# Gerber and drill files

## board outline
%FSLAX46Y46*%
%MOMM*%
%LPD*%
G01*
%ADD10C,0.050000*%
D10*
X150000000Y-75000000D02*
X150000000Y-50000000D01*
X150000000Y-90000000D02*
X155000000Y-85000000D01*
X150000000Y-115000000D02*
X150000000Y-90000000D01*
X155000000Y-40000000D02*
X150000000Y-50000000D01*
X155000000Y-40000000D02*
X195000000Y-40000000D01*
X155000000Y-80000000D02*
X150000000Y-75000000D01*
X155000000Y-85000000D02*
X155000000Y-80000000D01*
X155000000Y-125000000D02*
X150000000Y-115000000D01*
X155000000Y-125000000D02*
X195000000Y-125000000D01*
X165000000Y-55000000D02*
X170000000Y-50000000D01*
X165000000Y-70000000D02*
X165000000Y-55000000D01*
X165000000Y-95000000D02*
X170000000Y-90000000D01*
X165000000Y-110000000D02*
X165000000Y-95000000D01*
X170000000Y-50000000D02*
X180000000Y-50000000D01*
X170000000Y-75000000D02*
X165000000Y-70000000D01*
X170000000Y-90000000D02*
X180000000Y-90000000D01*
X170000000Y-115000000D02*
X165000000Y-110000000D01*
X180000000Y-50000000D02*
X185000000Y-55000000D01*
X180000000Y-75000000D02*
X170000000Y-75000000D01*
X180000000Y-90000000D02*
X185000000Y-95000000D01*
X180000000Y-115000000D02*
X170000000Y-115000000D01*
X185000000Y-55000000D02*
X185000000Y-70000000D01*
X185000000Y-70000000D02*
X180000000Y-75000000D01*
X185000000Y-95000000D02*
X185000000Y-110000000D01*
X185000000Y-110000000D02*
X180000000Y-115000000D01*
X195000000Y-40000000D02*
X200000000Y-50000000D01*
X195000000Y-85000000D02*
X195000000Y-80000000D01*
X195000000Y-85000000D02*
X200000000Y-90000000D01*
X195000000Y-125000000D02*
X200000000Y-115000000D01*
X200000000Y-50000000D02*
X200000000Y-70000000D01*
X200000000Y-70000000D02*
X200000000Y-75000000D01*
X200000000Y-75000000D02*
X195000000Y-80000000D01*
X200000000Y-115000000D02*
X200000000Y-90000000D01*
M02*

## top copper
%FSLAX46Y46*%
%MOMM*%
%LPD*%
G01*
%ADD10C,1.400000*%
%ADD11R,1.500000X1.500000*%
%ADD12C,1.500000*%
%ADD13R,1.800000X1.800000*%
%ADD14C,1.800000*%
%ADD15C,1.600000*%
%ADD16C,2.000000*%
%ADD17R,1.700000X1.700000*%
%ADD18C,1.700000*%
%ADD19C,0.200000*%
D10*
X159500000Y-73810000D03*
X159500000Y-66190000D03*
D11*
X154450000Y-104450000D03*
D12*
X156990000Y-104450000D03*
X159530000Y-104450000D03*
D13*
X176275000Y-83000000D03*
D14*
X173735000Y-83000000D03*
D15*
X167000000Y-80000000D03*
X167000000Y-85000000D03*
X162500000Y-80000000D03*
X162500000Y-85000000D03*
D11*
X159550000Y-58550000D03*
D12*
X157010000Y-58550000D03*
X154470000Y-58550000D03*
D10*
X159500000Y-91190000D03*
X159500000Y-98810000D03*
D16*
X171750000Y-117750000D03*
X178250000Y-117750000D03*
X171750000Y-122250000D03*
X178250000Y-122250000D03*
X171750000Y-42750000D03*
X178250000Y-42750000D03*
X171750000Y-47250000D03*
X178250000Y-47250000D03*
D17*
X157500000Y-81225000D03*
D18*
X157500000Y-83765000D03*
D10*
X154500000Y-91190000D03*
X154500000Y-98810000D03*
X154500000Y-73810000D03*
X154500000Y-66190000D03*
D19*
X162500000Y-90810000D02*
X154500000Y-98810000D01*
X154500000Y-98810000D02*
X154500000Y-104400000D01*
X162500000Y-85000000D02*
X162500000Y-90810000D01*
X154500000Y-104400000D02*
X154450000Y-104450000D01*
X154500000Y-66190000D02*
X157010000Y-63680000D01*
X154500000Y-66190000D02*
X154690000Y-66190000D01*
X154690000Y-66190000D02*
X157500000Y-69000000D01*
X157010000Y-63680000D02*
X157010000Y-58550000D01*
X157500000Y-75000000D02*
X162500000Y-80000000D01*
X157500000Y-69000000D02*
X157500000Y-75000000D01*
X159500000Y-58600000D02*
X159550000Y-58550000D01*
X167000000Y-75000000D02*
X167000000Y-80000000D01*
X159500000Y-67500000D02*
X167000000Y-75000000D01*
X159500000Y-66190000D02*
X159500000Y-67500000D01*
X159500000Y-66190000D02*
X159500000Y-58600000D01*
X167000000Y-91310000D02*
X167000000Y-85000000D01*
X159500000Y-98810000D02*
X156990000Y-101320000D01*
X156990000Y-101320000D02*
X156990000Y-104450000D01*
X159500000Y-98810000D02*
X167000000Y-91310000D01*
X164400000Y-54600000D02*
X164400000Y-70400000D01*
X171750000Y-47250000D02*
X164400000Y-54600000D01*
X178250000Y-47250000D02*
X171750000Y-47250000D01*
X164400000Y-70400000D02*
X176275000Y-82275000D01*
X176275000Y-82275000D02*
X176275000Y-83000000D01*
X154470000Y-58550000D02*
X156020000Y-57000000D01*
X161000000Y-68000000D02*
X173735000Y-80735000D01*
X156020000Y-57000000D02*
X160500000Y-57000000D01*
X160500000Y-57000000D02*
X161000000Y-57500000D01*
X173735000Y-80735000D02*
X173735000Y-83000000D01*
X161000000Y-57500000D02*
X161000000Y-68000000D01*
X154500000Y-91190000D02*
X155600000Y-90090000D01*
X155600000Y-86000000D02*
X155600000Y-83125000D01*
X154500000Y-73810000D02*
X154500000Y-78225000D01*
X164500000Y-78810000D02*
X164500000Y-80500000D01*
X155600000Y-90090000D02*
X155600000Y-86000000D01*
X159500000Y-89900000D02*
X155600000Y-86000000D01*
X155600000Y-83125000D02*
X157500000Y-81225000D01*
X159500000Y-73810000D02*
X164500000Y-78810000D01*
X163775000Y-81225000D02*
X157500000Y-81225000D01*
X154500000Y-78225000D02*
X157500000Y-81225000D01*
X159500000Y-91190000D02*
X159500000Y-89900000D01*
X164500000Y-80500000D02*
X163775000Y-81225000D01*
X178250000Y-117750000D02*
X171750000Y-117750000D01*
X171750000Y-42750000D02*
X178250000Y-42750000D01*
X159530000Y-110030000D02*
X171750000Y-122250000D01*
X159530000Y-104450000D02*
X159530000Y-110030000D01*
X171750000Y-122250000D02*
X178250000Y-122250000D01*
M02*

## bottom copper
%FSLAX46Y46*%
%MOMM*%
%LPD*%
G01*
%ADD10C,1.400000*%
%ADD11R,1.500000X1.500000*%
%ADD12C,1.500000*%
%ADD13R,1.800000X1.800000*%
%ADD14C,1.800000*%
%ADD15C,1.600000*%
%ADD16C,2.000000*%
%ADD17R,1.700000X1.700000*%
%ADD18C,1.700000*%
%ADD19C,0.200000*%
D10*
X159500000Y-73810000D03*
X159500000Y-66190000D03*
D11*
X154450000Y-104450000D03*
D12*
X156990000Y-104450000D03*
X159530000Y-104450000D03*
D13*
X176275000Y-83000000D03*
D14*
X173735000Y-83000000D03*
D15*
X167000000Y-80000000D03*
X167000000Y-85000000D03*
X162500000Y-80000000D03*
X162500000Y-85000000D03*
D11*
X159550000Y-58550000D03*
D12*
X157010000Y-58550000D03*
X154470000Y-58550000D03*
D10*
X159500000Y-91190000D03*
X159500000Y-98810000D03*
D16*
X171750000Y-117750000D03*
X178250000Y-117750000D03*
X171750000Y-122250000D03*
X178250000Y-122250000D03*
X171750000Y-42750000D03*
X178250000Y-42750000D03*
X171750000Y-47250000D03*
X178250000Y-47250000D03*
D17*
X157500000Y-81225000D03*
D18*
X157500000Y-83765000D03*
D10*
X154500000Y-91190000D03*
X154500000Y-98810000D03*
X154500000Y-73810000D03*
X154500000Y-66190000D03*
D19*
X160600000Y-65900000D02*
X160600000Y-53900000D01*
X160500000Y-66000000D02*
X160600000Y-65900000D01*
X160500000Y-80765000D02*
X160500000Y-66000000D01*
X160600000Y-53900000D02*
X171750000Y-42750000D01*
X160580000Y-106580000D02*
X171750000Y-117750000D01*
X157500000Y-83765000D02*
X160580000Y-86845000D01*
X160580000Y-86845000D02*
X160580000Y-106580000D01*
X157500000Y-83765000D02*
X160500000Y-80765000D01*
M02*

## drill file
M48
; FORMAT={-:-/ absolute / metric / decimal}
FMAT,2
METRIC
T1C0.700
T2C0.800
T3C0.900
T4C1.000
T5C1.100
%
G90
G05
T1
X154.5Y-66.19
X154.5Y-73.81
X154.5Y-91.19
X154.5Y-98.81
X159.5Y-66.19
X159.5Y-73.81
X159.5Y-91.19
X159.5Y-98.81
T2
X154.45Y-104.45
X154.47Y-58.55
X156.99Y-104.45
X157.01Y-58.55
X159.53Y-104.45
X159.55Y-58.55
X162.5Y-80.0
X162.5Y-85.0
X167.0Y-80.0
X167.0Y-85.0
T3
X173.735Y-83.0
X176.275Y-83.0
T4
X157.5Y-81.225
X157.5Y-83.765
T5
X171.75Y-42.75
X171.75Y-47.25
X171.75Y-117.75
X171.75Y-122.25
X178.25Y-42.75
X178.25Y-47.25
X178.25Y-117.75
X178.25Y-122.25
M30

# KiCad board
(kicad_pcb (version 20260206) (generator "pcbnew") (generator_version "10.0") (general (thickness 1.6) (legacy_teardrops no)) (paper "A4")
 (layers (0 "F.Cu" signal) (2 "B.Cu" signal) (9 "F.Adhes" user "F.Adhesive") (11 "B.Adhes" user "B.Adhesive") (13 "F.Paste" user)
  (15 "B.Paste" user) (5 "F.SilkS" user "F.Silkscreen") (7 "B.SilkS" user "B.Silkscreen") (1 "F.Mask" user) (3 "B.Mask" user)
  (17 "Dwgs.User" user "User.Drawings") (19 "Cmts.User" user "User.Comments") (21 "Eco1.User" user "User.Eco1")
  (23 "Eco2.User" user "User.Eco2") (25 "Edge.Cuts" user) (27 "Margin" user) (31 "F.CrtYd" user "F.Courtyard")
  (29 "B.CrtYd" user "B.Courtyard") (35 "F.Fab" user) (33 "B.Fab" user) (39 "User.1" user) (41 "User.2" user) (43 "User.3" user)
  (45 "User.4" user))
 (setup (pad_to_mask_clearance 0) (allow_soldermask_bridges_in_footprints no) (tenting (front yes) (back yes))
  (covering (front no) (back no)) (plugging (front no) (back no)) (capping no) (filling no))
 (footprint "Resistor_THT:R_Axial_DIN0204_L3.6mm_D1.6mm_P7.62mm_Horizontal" (layer "F.Cu") (at 159.5 73.81 90)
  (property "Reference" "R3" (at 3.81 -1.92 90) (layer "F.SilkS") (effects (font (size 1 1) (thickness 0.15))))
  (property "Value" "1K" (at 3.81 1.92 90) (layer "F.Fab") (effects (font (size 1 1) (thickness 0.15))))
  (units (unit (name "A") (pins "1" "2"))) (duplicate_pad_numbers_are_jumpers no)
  (pad "1" thru_hole circle (at 0 0 90) (size 1.4 1.4) (drill 0.7) (layers "*.Cu" "*.Mask") (remove_unused_layers no) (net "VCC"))
  (pad "2" thru_hole circle (at 7.62 0 90) (size 1.4 1.4) (drill 0.7) (layers "*.Cu" "*.Mask") (remove_unused_layers no) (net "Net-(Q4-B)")))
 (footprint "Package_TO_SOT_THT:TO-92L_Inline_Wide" (layer "F.Cu") (at 154.45 104.45)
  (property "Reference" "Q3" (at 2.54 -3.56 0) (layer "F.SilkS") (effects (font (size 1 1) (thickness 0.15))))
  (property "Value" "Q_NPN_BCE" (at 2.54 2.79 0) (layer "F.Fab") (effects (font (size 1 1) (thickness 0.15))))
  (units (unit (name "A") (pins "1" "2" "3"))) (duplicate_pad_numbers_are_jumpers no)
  (pad "1" thru_hole rect (at 0 0) (size 1.5 1.5) (drill 0.8) (layers "*.Cu" "*.Mask") (remove_unused_layers no) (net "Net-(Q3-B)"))
  (pad "2" thru_hole circle (at 2.54 0) (size 1.5 1.5) (drill 0.8) (layers "*.Cu" "*.Mask") (remove_unused_layers no) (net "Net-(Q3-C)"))
  (pad "3" thru_hole circle (at 5.08 0) (size 1.5 1.5) (drill 0.8) (layers "*.Cu" "*.Mask") (remove_unused_layers no) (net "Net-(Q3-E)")))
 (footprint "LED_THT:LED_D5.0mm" (layer "F.Cu") (at 176.275 83 180)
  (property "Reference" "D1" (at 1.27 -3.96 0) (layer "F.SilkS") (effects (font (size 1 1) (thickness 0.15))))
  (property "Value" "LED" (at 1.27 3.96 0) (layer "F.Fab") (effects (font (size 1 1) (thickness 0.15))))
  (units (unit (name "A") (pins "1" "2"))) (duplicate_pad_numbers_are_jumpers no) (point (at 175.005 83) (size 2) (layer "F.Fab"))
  (pad "1" thru_hole rect (at 0 0 180) (size 1.8 1.8) (drill 0.9) (layers "*.Cu" "*.Mask") (remove_unused_layers no) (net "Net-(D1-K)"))
  (pad "2" thru_hole circle (at 2.54 0 180) (size 1.8 1.8) (drill 0.9) (layers "*.Cu" "*.Mask") (remove_unused_layers no) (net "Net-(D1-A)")))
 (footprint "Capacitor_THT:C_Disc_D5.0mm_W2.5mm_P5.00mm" (layer "F.Cu") (at 167 80 -90)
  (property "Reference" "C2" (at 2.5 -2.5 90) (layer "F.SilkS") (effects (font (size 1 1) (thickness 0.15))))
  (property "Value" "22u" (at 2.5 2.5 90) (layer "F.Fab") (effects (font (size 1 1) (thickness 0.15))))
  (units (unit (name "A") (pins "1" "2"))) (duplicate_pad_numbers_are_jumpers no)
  (pad "1" thru_hole circle (at 0 0 270) (size 1.6 1.6) (drill 0.8) (layers "*.Cu" "*.Mask") (remove_unused_layers no) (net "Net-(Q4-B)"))
  (pad "2" thru_hole circle (at 5 0 270) (size 1.6 1.6) (drill 0.8) (layers "*.Cu" "*.Mask") (remove_unused_layers no) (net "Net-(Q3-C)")))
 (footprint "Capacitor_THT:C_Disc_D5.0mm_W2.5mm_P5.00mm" (layer "F.Cu") (at 162.5 80 -90)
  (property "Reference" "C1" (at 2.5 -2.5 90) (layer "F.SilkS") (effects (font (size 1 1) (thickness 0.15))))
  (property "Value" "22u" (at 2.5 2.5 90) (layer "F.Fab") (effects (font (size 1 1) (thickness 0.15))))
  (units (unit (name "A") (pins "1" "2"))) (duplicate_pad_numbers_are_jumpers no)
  (pad "1" thru_hole circle (at 0 0 270) (size 1.6 1.6) (drill 0.8) (layers "*.Cu" "*.Mask") (remove_unused_layers no) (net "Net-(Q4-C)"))
  (pad "2" thru_hole circle (at 5 0 270) (size 1.6 1.6) (drill 0.8) (layers "*.Cu" "*.Mask") (remove_unused_layers no) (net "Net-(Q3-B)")))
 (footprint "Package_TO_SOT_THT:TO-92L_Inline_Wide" (layer "F.Cu") (at 159.55 58.55 180)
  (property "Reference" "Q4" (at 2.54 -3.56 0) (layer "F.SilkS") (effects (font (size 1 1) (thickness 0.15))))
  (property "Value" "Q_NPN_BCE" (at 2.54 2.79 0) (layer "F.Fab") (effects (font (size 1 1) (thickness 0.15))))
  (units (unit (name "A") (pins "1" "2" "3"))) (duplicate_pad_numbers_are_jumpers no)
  (pad "1" thru_hole rect (at 0 0 180) (size 1.5 1.5) (drill 0.8) (layers "*.Cu" "*.Mask") (remove_unused_layers no) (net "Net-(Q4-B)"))
  (pad "2" thru_hole circle (at 2.54 0 180) (size 1.5 1.5) (drill 0.8) (layers "*.Cu" "*.Mask") (remove_unused_layers no) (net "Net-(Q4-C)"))
  (pad "3" thru_hole circle (at 5.08 0 180) (size 1.5 1.5) (drill 0.8) (layers "*.Cu" "*.Mask") (remove_unused_layers no) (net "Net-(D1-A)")))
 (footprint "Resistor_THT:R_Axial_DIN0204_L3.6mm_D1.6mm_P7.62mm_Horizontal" (layer "F.Cu") (at 159.5 91.19 -90)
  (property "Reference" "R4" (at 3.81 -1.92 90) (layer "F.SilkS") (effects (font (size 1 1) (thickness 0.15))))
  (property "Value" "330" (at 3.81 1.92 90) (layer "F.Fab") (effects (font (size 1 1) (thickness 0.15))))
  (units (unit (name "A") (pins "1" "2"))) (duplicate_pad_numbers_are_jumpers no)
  (pad "1" thru_hole circle (at 0 0 270) (size 1.4 1.4) (drill 0.7) (layers "*.Cu" "*.Mask") (remove_unused_layers no) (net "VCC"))
  (pad "2" thru_hole circle (at 7.62 0 270) (size 1.4 1.4) (drill 0.7) (layers "*.Cu" "*.Mask") (remove_unused_layers no) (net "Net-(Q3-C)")))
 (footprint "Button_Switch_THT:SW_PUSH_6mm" (layer "F.Cu") (at 171.75 117.75)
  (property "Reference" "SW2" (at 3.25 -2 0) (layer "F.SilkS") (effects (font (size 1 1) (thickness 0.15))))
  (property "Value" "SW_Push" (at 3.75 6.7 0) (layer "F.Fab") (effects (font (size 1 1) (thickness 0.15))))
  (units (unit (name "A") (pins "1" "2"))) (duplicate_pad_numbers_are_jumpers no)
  (pad "1" thru_hole circle (at 0 0 90) (size 2 2) (drill 1.1) (layers "*.Cu" "*.Mask") (remove_unused_layers no) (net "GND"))
  (pad "1" thru_hole circle (at 6.5 0 90) (size 2 2) (drill 1.1) (layers "*.Cu" "*.Mask") (remove_unused_layers no) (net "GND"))
  (pad "2" thru_hole circle (at 0 4.5 90) (size 2 2) (drill 1.1) (layers "*.Cu" "*.Mask") (remove_unused_layers no) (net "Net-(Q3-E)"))
  (pad "2" thru_hole circle (at 6.5 4.5 90) (size 2 2) (drill 1.1) (layers "*.Cu" "*.Mask") (remove_unused_layers no) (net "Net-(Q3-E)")))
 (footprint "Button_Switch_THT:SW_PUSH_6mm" (layer "F.Cu") (at 171.75 42.75)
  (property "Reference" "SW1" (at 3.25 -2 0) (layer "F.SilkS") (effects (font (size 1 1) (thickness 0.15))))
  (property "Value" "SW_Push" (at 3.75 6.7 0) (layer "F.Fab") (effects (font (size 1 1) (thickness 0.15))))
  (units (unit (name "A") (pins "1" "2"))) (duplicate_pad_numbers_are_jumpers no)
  (pad "1" thru_hole circle (at 0 0 90) (size 2 2) (drill 1.1) (layers "*.Cu" "*.Mask") (remove_unused_layers no) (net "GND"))
  (pad "1" thru_hole circle (at 6.5 0 90) (size 2 2) (drill 1.1) (layers "*.Cu" "*.Mask") (remove_unused_layers no) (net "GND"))
  (pad "2" thru_hole circle (at 0 4.5 90) (size 2 2) (drill 1.1) (layers "*.Cu" "*.Mask") (remove_unused_layers no) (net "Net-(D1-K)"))
  (pad "2" thru_hole circle (at 6.5 4.5 90) (size 2 2) (drill 1.1) (layers "*.Cu" "*.Mask") (remove_unused_layers no) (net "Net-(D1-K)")))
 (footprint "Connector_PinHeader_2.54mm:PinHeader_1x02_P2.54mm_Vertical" (layer "F.Cu") (at 157.5 81.225)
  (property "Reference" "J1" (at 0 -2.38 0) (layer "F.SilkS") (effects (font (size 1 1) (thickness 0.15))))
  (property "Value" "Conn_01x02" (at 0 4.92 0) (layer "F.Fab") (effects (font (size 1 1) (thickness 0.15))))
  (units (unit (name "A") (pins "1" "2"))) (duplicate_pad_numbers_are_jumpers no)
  (pad "1" thru_hole rect (at 0 0) (size 1.7 1.7) (drill 1) (layers "*.Cu" "*.Mask") (remove_unused_layers no) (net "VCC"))
  (pad "2" thru_hole circle (at 0 2.54) (size 1.7 1.7) (drill 1) (layers "*.Cu" "*.Mask") (remove_unused_layers no) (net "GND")))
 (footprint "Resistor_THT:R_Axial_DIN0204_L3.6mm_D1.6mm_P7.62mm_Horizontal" (layer "F.Cu") (at 154.5 91.19 -90)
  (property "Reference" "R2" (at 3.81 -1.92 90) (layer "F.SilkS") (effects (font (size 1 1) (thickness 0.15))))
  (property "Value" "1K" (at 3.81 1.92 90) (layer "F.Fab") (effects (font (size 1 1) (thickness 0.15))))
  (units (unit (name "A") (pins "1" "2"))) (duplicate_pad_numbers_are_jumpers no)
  (pad "1" thru_hole circle (at 0 0 270) (size 1.4 1.4) (drill 0.7) (layers "*.Cu" "*.Mask") (remove_unused_layers no) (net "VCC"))
  (pad "2" thru_hole circle (at 7.62 0 270) (size 1.4 1.4) (drill 0.7) (layers "*.Cu" "*.Mask") (remove_unused_layers no) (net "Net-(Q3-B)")))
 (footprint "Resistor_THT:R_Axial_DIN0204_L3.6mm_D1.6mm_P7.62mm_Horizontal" (layer "F.Cu") (at 154.5 73.81 90)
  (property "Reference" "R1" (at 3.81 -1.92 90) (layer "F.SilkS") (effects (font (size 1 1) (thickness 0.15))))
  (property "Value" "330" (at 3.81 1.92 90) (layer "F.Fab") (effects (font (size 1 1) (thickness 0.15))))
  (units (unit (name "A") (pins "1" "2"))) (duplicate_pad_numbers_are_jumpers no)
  (pad "1" thru_hole circle (at 0 0 90) (size 1.4 1.4) (drill 0.7) (layers "*.Cu" "*.Mask") (remove_unused_layers no) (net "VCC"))
  (pad "2" thru_hole circle (at 7.62 0 90) (size 1.4 1.4) (drill 0.7) (layers "*.Cu" "*.Mask") (remove_unused_layers no) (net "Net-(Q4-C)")))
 (gr_line (start 150 75) (end 150 50) (stroke (width 0.05) (type default)) (layer "Edge.Cuts"))
 (gr_line (start 150 90) (end 155 85) (stroke (width 0.05) (type default)) (layer "Edge.Cuts"))
 (gr_line (start 150 115) (end 150 90) (stroke (width 0.05) (type default)) (layer "Edge.Cuts"))
 (gr_line (start 155 40) (end 150 50) (stroke (width 0.05) (type default)) (layer "Edge.Cuts"))
 (gr_line (start 155 40) (end 195 40) (stroke (width 0.05) (type default)) (layer "Edge.Cuts"))
 (gr_line (start 155 80) (end 150 75) (stroke (width 0.05) (type default)) (layer "Edge.Cuts"))
 (gr_line (start 155 85) (end 155 80) (stroke (width 0.05) (type default)) (layer "Edge.Cuts"))
 (gr_line (start 155 125) (end 150 115) (stroke (width 0.05) (type default)) (layer "Edge.Cuts"))
 (gr_line (start 155 125) (end 195 125) (stroke (width 0.05) (type default)) (layer "Edge.Cuts"))
 (gr_line (start 165 55) (end 170 50) (stroke (width 0.05) (type default)) (layer "Edge.Cuts"))
 (gr_line (start 165 70) (end 165 55) (stroke (width 0.05) (type default)) (layer "Edge.Cuts"))
 (gr_line (start 165 95) (end 170 90) (stroke (width 0.05) (type default)) (layer "Edge.Cuts"))
 (gr_line (start 165 110) (end 165 95) (stroke (width 0.05) (type default)) (layer "Edge.Cuts"))
 (gr_line (start 170 50) (end 180 50) (stroke (width 0.05) (type default)) (layer "Edge.Cuts"))
 (gr_line (start 170 75) (end 165 70) (stroke (width 0.05) (type default)) (layer "Edge.Cuts"))
 (gr_line (start 170 90) (end 180 90) (stroke (width 0.05) (type default)) (layer "Edge.Cuts"))
 (gr_line (start 170 115) (end 165 110) (stroke (width 0.05) (type default)) (layer "Edge.Cuts"))
 (gr_line (start 180 50) (end 185 55) (stroke (width 0.05) (type default)) (layer "Edge.Cuts"))
 (gr_line (start 180 75) (end 170 75) (stroke (width 0.05) (type default)) (layer "Edge.Cuts"))
 (gr_line (start 180 90) (end 185 95) (stroke (width 0.05) (type default)) (layer "Edge.Cuts"))
 (gr_line (start 180 115) (end 170 115) (stroke (width 0.05) (type default)) (layer "Edge.Cuts"))
 (gr_line (start 185 55) (end 185 70) (stroke (width 0.05) (type default)) (layer "Edge.Cuts"))
 (gr_line (start 185 70) (end 180 75) (stroke (width 0.05) (type default)) (layer "Edge.Cuts"))
 (gr_line (start 185 95) (end 185 110) (stroke (width 0.05) (type default)) (layer "Edge.Cuts"))
 (gr_line (start 185 110) (end 180 115) (stroke (width 0.05) (type default)) (layer "Edge.Cuts"))
 (gr_line (start 195 40) (end 200 50) (stroke (width 0.05) (type default)) (layer "Edge.Cuts"))
 (gr_line (start 195 85) (end 195 80) (stroke (width 0.05) (type default)) (layer "Edge.Cuts"))
 (gr_line (start 195 85) (end 200 90) (stroke (width 0.05) (type default)) (layer "Edge.Cuts"))
 (gr_line (start 195 125) (end 200 115) (stroke (width 0.05) (type default)) (layer "Edge.Cuts"))
 (gr_line (start 200 50) (end 200 70) (stroke (width 0.05) (type default)) (layer "Edge.Cuts"))
 (gr_line (start 200 70) (end 200 75) (stroke (width 0.05) (type default)) (layer "Edge.Cuts"))
 (gr_line (start 200 75) (end 195 80) (stroke (width 0.05) (type default)) (layer "Edge.Cuts"))
 (gr_line (start 200 115) (end 200 90) (stroke (width 0.05) (type default)) (layer "Edge.Cuts"))
 (segment (start 162.5 90.81) (end 154.5 98.81) (width 0.2) (layer "F.Cu") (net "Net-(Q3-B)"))
 (segment (start 154.5 98.81) (end 154.5 104.4) (width 0.2) (layer "F.Cu") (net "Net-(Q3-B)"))
 (segment (start 162.5 85) (end 162.5 90.81) (width 0.2) (layer "F.Cu") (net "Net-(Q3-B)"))
 (segment (start 154.5 104.4) (end 154.45 104.45) (width 0.2) (layer "F.Cu") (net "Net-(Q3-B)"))
 (segment (start 154.5 66.19) (end 157.01 63.68) (width 0.2) (layer "F.Cu") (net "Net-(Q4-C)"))
 (segment (start 154.5 66.19) (end 154.69 66.19) (width 0.2) (layer "F.Cu") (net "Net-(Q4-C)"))
 (segment (start 154.69 66.19) (end 157.5 69) (width 0.2) (layer "F.Cu") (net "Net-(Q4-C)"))
 (segment (start 157.01 63.68) (end 157.01 58.55) (width 0.2) (layer "F.Cu") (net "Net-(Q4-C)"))
 (segment (start 157.5 75) (end 162.5 80) (width 0.2) (layer "F.Cu") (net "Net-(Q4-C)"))
 (segment (start 157.5 69) (end 157.5 75) (width 0.2) (layer "F.Cu") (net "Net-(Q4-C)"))
 (segment (start 159.5 58.6) (end 159.55 58.55) (width 0.2) (layer "F.Cu") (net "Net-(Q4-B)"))
 (segment (start 167 75) (end 167 80) (width 0.2) (layer "F.Cu") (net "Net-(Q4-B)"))
 (segment (start 159.5 67.5) (end 167 75) (width 0.2) (layer "F.Cu") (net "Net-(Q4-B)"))
 (segment (start 159.5 66.19) (end 159.5 67.5) (width 0.2) (layer "F.Cu") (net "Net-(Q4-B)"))
 (segment (start 159.5 66.19) (end 159.5 58.6) (width 0.2) (layer "F.Cu") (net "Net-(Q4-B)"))
 (segment (start 167 91.31) (end 167 85) (width 0.2) (layer "F.Cu") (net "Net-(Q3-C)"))
 (segment (start 159.5 98.81) (end 156.99 101.32) (width 0.2) (layer "F.Cu") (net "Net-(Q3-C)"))
 (segment (start 156.99 101.32) (end 156.99 104.45) (width 0.2) (layer "F.Cu") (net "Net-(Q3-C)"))
 (segment (start 159.5 98.81) (end 167 91.31) (width 0.2) (layer "F.Cu") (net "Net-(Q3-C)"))
 (segment (start 164.4 54.6) (end 164.4 70.4) (width 0.2) (layer "F.Cu") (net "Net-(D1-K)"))
 (segment (start 171.75 47.25) (end 164.4 54.6) (width 0.2) (layer "F.Cu") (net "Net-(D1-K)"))
 (segment (start 178.25 47.25) (end 171.75 47.25) (width 0.2) (layer "F.Cu") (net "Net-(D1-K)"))
 (segment (start 164.4 70.4) (end 176.275 82.275) (width 0.2) (layer "F.Cu") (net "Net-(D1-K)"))
 (segment (start 176.275 82.275) (end 176.275 83) (width 0.2) (layer "F.Cu") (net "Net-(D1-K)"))
 (segment (start 154.47 58.55) (end 156.02 57) (width 0.2) (layer "F.Cu") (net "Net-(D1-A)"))
 (segment (start 161 68) (end 173.735 80.735) (width 0.2) (layer "F.Cu") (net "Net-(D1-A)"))
 (segment (start 156.02 57) (end 160.5 57) (width 0.2) (layer "F.Cu") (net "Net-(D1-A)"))
 (segment (start 160.5 57) (end 161 57.5) (width 0.2) (layer "F.Cu") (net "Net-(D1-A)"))
 (segment (start 173.735 80.735) (end 173.735 83) (width 0.2) (layer "F.Cu") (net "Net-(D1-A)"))
 (segment (start 161 57.5) (end 161 68) (width 0.2) (layer "F.Cu") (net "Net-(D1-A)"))
 (segment (start 154.5 91.19) (end 155.6 90.09) (width 0.2) (layer "F.Cu") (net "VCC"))
 (segment (start 155.6 86) (end 155.6 83.125) (width 0.2) (layer "F.Cu") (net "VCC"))
 (segment (start 154.5 73.81) (end 154.5 78.225) (width 0.2) (layer "F.Cu") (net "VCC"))
 (segment (start 164.5 78.81) (end 164.5 80.5) (width 0.2) (layer "F.Cu") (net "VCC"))
 (segment (start 155.6 90.09) (end 155.6 86) (width 0.2) (layer "F.Cu") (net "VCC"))
 (segment (start 159.5 89.9) (end 155.6 86) (width 0.2) (layer "F.Cu") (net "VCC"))
 (segment (start 155.6 83.125) (end 157.5 81.225) (width 0.2) (layer "F.Cu") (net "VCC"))
 (segment (start 159.5 73.81) (end 164.5 78.81) (width 0.2) (layer "F.Cu") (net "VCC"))
 (segment (start 163.775 81.225) (end 157.5 81.225) (width 0.2) (layer "F.Cu") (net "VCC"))
 (segment (start 154.5 78.225) (end 157.5 81.225) (width 0.2) (layer "F.Cu") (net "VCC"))
 (segment (start 159.5 91.19) (end 159.5 89.9) (width 0.2) (layer "F.Cu") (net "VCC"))
 (segment (start 164.5 80.5) (end 163.775 81.225) (width 0.2) (layer "F.Cu") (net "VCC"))
 (segment (start 178.25 117.75) (end 171.75 117.75) (width 0.2) (layer "F.Cu") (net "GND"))
 (segment (start 171.75 42.75) (end 178.25 42.75) (width 0.2) (layer "F.Cu") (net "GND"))
 (segment (start 160.6 65.9) (end 160.6 53.9) (width 0.2) (layer "B.Cu") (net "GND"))
 (segment (start 160.5 66) (end 160.6 65.9) (width 0.2) (layer "B.Cu") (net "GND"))
 (segment (start 160.5 80.765) (end 160.5 66) (width 0.2) (layer "B.Cu") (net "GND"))
 (segment (start 160.6 53.9) (end 171.75 42.75) (width 0.2) (layer "B.Cu") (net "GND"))
 (segment (start 160.58 106.58) (end 171.75 117.75) (width 0.2) (layer "B.Cu") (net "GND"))
 (segment (start 157.5 83.765) (end 160.58 86.845) (width 0.2) (layer "B.Cu") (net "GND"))
 (segment (start 160.58 86.845) (end 160.58 106.58) (width 0.2) (layer "B.Cu") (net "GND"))
 (segment (start 157.5 83.765) (end 160.5 80.765) (width 0.2) (layer "B.Cu") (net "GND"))
 (segment (start 159.53 110.03) (end 171.75 122.25) (width 0.2) (layer "F.Cu") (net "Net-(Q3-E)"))
 (segment (start 159.53 104.45) (end 159.53 110.03) (width 0.2) (layer "F.Cu") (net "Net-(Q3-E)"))
 (segment (start 171.75 122.25) (end 178.25 122.25) (width 0.2) (layer "F.Cu") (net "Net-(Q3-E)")))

